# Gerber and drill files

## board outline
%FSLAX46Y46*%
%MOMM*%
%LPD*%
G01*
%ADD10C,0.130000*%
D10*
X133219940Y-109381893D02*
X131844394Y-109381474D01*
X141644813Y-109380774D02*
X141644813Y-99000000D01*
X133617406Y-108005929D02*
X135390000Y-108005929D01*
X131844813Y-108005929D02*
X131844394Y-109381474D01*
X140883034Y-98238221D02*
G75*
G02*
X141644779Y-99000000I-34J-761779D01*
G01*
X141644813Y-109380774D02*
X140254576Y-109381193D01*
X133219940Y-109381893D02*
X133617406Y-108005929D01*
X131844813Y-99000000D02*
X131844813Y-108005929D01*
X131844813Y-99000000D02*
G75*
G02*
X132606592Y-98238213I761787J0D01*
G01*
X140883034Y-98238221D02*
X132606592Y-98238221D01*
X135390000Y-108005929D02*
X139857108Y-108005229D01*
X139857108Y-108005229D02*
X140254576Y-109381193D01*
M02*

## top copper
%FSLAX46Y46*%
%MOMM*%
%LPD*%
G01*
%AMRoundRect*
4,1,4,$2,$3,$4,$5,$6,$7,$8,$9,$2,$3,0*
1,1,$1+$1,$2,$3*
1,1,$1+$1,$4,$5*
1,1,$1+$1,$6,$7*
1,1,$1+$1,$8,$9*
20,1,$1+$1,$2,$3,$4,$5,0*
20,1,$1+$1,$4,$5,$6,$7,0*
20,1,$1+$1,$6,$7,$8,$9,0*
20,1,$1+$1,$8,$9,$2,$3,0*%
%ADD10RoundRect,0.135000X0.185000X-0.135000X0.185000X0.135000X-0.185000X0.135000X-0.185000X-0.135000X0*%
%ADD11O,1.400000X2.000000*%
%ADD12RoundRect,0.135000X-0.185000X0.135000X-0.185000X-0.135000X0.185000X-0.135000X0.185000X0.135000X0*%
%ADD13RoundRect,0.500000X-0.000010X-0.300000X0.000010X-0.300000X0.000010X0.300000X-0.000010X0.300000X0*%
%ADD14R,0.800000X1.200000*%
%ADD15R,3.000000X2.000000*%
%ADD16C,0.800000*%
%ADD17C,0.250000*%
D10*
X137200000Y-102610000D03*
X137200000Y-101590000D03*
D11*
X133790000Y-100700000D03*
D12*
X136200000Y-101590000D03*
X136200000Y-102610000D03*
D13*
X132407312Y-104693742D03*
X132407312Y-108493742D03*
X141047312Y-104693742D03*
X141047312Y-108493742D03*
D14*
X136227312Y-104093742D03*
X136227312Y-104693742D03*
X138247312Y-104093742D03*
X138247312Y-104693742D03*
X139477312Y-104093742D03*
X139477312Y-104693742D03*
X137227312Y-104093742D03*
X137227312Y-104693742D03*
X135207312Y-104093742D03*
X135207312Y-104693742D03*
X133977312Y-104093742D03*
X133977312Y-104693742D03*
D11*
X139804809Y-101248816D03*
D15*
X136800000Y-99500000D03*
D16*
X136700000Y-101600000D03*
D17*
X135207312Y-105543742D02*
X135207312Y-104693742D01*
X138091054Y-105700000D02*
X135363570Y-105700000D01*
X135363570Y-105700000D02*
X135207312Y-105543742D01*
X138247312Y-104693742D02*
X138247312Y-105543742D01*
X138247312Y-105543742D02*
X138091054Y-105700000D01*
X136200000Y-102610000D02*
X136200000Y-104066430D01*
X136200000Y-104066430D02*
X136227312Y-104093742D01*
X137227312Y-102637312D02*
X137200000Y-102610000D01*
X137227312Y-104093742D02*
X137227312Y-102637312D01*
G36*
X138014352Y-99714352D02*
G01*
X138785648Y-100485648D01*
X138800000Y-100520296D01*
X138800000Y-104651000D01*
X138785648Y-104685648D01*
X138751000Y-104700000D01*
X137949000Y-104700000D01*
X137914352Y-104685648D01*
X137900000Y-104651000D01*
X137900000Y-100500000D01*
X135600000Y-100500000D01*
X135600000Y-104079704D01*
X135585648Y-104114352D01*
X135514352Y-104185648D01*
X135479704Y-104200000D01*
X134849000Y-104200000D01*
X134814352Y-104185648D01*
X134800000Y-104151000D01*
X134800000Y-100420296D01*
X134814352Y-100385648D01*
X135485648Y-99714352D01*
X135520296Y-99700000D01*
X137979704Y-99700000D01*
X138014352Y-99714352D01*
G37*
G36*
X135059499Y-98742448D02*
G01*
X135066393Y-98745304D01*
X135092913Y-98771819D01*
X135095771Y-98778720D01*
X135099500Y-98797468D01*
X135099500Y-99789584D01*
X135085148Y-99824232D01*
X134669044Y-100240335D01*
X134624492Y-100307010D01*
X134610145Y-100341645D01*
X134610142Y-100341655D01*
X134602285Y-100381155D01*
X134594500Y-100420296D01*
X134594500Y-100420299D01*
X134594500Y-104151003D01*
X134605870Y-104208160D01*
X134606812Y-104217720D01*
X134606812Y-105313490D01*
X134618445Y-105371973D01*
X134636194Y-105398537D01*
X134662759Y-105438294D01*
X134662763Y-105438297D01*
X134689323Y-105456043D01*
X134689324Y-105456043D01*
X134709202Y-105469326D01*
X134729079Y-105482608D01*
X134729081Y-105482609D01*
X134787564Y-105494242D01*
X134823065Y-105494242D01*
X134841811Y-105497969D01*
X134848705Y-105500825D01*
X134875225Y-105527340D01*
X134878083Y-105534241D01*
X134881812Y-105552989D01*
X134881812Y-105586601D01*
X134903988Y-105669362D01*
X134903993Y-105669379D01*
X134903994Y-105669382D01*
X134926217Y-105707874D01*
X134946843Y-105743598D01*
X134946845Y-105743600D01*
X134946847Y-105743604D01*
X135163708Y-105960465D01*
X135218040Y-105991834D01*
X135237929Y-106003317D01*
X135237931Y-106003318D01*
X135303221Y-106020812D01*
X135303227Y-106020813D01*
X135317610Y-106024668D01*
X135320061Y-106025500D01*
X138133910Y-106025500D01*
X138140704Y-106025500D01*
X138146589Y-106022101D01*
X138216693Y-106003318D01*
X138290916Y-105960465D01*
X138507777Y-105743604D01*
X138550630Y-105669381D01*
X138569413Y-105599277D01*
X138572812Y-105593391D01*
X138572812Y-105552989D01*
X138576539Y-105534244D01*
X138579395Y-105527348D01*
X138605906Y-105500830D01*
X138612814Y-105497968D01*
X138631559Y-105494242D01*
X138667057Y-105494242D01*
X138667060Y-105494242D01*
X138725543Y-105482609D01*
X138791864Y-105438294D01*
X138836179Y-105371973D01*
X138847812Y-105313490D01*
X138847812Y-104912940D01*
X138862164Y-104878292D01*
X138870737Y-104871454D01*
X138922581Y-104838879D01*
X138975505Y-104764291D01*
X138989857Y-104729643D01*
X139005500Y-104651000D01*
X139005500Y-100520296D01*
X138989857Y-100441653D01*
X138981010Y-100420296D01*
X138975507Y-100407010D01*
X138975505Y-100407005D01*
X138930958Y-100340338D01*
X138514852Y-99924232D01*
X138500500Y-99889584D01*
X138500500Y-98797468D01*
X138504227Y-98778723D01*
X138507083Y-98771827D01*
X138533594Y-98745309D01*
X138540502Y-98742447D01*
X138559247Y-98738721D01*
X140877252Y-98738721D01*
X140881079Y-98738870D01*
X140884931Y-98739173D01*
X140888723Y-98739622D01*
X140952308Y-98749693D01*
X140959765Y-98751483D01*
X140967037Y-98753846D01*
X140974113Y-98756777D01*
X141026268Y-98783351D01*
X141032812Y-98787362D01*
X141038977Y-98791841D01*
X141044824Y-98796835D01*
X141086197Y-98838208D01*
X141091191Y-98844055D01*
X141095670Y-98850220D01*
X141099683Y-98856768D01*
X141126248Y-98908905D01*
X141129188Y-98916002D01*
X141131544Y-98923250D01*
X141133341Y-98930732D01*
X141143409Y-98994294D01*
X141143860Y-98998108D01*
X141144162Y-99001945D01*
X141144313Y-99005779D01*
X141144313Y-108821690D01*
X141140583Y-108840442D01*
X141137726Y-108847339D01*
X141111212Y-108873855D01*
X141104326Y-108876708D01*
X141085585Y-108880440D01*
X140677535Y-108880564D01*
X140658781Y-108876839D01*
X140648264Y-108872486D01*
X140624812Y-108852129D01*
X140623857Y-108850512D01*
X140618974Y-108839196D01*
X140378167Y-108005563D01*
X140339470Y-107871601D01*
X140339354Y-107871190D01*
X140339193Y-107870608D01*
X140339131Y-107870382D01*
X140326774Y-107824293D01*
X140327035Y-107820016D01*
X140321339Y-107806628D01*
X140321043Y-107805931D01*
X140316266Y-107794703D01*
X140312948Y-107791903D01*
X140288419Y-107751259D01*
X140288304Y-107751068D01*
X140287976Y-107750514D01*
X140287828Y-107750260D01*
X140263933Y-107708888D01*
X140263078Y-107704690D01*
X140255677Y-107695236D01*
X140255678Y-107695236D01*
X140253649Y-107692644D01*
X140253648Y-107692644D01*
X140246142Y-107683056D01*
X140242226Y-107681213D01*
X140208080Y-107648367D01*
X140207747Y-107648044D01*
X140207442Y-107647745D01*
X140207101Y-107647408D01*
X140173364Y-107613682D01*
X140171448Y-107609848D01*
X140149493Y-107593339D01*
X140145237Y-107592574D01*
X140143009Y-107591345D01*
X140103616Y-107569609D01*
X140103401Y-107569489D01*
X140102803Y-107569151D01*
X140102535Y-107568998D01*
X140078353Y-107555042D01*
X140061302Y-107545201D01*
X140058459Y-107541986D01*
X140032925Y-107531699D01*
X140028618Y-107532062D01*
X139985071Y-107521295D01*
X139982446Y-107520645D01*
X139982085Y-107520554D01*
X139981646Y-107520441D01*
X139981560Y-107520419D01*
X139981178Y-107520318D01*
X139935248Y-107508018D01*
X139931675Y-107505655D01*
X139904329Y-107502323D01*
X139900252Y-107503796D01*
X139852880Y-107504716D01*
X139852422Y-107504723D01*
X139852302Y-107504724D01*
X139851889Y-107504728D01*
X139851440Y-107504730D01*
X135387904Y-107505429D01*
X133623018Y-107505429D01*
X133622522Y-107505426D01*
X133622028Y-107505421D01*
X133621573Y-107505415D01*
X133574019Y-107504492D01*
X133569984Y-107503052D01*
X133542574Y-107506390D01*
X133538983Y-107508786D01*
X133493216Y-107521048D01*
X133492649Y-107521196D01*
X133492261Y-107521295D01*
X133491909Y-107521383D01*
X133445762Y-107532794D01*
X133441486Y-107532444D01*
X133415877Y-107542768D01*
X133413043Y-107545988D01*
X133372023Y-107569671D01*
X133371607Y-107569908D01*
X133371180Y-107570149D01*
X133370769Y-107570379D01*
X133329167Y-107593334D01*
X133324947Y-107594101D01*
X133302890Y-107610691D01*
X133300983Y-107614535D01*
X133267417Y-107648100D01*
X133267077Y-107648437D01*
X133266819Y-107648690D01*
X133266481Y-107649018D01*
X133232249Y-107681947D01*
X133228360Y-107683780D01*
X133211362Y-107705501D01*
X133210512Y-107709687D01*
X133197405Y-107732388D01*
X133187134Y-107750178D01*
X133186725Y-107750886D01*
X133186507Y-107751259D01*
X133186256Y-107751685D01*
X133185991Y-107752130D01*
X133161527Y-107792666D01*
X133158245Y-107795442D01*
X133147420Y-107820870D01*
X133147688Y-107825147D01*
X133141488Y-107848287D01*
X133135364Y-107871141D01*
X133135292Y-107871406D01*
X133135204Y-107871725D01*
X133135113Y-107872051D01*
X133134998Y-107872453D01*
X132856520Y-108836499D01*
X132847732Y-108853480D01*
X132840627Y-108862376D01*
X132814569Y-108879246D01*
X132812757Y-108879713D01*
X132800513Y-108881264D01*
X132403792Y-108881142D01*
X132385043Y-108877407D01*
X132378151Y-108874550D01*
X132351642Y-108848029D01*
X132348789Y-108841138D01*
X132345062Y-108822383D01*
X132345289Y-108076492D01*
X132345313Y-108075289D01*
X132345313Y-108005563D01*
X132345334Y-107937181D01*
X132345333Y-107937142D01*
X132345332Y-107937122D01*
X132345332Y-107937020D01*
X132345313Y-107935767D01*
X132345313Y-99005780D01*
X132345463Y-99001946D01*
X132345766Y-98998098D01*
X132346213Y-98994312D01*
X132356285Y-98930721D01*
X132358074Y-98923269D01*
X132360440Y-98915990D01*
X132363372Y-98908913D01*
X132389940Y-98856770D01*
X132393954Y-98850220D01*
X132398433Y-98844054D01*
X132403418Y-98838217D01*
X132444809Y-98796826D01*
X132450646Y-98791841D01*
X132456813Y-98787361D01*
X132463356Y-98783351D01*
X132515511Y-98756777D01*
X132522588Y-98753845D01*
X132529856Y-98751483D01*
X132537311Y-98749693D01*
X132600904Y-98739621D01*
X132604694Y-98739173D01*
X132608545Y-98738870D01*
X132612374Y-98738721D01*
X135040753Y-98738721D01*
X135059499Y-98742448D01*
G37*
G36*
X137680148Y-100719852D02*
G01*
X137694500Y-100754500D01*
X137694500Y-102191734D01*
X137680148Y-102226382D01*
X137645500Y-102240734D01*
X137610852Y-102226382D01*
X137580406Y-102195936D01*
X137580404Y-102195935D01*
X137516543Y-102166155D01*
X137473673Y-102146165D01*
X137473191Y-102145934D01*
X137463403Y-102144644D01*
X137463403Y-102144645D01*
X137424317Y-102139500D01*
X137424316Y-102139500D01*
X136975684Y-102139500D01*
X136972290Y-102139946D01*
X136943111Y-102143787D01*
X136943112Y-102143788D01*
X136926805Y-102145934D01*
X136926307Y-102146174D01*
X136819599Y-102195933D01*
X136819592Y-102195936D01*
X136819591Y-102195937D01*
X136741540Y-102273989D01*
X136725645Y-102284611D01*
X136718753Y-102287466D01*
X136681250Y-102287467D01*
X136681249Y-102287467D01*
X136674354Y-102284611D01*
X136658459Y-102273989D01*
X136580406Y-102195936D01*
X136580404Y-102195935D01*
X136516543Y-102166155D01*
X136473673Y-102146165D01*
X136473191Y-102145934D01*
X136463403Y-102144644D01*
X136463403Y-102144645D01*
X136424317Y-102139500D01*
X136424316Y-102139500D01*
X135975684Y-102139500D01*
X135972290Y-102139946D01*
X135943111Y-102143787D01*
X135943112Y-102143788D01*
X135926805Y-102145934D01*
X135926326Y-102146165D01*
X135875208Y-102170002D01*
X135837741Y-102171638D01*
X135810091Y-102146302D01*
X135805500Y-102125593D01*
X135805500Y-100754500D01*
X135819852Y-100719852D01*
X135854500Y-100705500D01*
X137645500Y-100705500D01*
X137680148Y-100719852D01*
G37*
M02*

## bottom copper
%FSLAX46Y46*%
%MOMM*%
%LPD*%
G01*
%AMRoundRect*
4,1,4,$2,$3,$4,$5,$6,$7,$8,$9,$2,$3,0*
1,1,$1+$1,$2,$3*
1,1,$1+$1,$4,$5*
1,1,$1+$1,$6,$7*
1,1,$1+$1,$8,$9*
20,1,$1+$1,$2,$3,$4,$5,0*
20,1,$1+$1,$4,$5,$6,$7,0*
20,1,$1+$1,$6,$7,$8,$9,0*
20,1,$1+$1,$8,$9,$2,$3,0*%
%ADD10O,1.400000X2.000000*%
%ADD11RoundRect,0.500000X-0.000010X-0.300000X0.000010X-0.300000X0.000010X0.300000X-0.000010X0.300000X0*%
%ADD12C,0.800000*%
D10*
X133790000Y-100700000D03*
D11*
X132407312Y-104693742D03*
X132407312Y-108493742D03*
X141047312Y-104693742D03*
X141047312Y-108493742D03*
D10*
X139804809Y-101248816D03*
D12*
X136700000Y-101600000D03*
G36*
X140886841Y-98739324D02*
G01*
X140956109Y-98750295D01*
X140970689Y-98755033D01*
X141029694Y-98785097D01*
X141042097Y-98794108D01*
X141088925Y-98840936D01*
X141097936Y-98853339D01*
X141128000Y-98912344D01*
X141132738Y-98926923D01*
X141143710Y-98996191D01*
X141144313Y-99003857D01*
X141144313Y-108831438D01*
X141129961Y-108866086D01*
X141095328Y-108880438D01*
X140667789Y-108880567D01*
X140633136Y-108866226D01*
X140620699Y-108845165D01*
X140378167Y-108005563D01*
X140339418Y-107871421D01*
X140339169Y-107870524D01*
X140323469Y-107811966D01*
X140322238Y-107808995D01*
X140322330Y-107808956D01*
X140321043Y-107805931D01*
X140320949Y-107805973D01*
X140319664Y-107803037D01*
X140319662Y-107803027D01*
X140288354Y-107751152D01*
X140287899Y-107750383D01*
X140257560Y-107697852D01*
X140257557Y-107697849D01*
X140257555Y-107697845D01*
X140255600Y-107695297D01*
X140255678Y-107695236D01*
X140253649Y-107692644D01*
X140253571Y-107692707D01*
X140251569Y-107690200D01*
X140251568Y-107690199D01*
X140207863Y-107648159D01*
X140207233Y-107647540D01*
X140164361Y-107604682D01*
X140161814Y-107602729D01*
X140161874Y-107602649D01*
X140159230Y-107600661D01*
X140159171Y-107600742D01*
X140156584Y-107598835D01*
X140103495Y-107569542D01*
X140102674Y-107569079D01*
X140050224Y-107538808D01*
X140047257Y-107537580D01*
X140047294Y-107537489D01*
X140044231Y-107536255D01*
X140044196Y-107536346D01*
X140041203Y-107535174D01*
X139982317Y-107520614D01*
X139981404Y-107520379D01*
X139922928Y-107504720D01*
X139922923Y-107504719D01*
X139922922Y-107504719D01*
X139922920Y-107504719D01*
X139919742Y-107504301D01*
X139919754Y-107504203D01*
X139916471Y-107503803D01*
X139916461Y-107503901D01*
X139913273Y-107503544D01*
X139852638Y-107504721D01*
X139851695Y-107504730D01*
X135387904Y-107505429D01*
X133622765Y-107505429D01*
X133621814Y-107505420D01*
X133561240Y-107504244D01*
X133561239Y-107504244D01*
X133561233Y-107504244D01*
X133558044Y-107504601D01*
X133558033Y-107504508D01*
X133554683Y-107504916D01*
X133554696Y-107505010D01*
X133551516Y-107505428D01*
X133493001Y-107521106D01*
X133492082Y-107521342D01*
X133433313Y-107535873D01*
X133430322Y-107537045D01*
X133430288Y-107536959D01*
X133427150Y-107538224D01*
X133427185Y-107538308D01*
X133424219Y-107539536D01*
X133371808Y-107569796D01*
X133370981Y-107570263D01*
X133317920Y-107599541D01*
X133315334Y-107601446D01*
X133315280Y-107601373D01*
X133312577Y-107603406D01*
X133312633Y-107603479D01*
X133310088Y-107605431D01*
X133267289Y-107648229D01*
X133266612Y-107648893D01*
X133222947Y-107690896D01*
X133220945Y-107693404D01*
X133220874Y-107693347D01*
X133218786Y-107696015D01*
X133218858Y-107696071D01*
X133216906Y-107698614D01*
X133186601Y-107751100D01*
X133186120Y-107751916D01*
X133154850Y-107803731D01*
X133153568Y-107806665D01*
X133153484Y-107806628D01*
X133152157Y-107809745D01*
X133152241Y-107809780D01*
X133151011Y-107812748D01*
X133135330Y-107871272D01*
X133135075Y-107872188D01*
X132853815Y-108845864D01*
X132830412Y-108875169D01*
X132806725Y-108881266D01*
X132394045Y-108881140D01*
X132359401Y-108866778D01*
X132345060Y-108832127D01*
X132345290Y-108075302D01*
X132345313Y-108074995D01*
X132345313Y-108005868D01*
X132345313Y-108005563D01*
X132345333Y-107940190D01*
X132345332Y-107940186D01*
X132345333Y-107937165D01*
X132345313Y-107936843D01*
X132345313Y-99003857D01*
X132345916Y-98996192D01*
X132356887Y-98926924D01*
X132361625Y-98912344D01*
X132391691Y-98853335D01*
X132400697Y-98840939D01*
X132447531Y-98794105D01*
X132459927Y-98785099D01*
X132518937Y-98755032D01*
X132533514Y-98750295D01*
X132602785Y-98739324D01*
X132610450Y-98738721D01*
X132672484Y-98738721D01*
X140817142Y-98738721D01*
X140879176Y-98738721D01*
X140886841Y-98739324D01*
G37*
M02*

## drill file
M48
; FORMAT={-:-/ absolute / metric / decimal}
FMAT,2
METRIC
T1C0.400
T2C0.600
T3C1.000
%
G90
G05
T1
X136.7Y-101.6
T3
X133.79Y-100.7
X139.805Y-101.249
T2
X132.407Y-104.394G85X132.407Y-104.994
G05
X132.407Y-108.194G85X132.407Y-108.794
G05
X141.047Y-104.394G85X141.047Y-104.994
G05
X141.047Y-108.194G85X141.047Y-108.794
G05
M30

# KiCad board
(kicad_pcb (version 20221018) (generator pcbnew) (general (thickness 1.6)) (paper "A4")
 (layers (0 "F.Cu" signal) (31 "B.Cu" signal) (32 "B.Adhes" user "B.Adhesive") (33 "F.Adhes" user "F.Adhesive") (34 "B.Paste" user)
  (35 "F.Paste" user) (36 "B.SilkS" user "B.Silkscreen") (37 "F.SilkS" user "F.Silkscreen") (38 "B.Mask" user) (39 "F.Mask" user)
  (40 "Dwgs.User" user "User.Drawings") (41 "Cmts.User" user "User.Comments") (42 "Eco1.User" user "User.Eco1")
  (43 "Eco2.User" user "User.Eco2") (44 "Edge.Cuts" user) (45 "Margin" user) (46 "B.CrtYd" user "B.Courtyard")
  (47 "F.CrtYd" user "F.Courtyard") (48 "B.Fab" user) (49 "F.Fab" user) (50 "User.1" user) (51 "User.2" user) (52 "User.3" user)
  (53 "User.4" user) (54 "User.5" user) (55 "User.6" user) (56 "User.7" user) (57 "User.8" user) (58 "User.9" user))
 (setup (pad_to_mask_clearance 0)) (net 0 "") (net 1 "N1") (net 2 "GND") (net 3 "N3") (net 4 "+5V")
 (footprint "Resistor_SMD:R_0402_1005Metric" (layer "F.Cu") (at 137.2 102.1 90)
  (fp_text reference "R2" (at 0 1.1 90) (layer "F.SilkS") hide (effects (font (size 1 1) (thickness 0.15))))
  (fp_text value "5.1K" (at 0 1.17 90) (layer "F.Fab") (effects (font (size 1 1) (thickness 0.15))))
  (pad "1" smd roundrect (at -0.51 0 90) (size 0.54 0.64) (layers "F.Cu" "F.Paste" "F.Mask") (roundrect_rratio 0.25) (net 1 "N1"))
  (pad "2" smd roundrect (at 0.51 0 90) (size 0.54 0.64) (layers "F.Cu" "F.Paste" "F.Mask") (roundrect_rratio 0.25) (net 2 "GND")))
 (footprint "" (layer "F.Cu") (at 133.79 100.7 -90)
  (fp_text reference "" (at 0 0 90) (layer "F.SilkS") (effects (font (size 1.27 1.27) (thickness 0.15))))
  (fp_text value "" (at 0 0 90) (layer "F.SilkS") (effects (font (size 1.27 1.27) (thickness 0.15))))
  (pad "1" thru_hole oval (at 0 0 90) (size 2 1.4) (drill 1) (layers "*.Cu" "*.Mask") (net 2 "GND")))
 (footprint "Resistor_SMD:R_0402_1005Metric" (layer "F.Cu") (at 136.2 102.1 -90)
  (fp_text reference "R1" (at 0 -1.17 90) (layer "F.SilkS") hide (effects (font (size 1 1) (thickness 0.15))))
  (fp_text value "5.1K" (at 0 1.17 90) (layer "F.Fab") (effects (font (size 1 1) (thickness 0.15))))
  (pad "1" smd roundrect (at -0.51 0 270) (size 0.54 0.64) (layers "F.Cu" "F.Paste" "F.Mask") (roundrect_rratio 0.25) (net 2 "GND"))
  (pad "2" smd roundrect (at 0.51 0 270) (size 0.54 0.64) (layers "F.Cu" "F.Paste" "F.Mask") (roundrect_rratio 0.25) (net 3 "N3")))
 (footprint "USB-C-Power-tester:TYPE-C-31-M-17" (layer "F.Cu") (at 136.727312 108.493742)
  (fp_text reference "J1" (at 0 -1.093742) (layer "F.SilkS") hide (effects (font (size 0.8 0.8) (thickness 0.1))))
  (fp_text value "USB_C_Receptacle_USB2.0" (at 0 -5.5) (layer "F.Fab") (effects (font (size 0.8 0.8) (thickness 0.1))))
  (pad "1" thru_hole roundrect (at -4.32 -3.8) (size 1 1.6) (drill oval 0.6 1.2) (layers "*.Cu" "*.Mask") (roundrect_rratio 0.5)
   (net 2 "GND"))
  (pad "1" thru_hole roundrect (at -4.32 0) (size 1 1.6) (drill oval 0.6 1.2) (layers "*.Cu" "*.Mask") (roundrect_rratio 0.5) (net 2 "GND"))
  (pad "1" thru_hole roundrect (at 4.32 -3.8) (size 1 1.6) (drill oval 0.6 1.2) (layers "*.Cu" "*.Mask") (roundrect_rratio 0.5)
   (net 2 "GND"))
  (pad "1" thru_hole roundrect (at 4.32 0) (size 1 1.6) (drill oval 0.6 1.2) (layers "*.Cu" "*.Mask") (roundrect_rratio 0.5) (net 2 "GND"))
  (pad "A5" smd rect (at -0.5 -4.4) (size 0.8 1.2) (layers "F.Cu" "F.Paste" "F.Mask") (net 3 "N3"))
  (pad "A5" smd rect (at -0.5 -3.8) (size 0.8 1.2) (layers "F.Cu" "F.Paste" "F.Mask") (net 3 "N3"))
  (pad "A9" smd rect (at 1.52 -4.4) (size 0.8 1.2) (layers "F.Cu" "F.Paste" "F.Mask") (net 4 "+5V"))
  (pad "A9" smd rect (at 1.52 -3.8) (size 0.8 1.2) (layers "F.Cu" "F.Paste" "F.Mask") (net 4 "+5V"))
  (pad "A12" smd rect (at 2.75 -4.4) (size 0.8 1.2) (layers "F.Cu" "F.Paste" "F.Mask") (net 2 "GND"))
  (pad "A12" smd rect (at 2.75 -3.8) (size 0.8 1.2) (layers "F.Cu" "F.Paste" "F.Mask") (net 2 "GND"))
  (pad "B5" smd rect (at 0.5 -4.4) (size 0.8 1.2) (layers "F.Cu" "F.Paste" "F.Mask") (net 1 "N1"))
  (pad "B5" smd rect (at 0.5 -3.8) (size 0.8 1.2) (layers "F.Cu" "F.Paste" "F.Mask") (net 1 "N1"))
  (pad "B9" smd rect (at -1.52 -4.4) (size 0.8 1.2) (layers "F.Cu" "F.Paste" "F.Mask") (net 4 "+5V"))
  (pad "B9" smd rect (at -1.52 -3.8) (size 0.8 1.2) (layers "F.Cu" "F.Paste" "F.Mask") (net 4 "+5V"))
  (pad "B12" smd rect (at -2.75 -4.4) (size 0.8 1.2) (layers "F.Cu" "F.Paste" "F.Mask") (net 2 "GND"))
  (pad "B12" smd rect (at -2.75 -3.8) (size 0.8 1.2) (layers "F.Cu" "F.Paste" "F.Mask") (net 2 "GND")))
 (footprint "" (layer "F.Cu") (at 139.804809 101.248816 -90)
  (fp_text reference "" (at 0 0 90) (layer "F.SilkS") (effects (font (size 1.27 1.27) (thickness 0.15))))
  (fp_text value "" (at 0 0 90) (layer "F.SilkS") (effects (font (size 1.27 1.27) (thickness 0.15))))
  (pad "1" thru_hole oval (at 0 0 270) (size 2 1.4) (drill 1) (layers "*.Cu" "*.Mask") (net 2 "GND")))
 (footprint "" (layer "F.Cu") (at 136.8 99.5 90)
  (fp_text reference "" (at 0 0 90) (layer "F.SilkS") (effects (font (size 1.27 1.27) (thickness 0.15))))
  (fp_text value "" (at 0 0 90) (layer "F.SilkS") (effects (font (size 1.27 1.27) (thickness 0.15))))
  (pad "" smd rect (at 0 0 90) (size 2 3) (layers "F.Cu" "F.Paste" "F.Mask") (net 4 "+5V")))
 (gr_line (start 133.21994 109.381893) (end 131.844394 109.381474) (stroke (width 0.13) (type solid)) (layer "Edge.Cuts"))
 (gr_line (start 141.644813 109.380774) (end 141.644813 99) (stroke (width 0.13) (type solid)) (layer "Edge.Cuts"))
 (gr_line (start 133.617406 108.005929) (end 135.39 108.005929) (stroke (width 0.13) (type solid)) (layer "Edge.Cuts"))
 (gr_line (start 131.844813 108.005929) (end 131.844394 109.381474) (stroke (width 0.13) (type solid)) (layer "Edge.Cuts"))
 (gr_arc (start 140.883034 98.238221) (mid 141.421693 98.461341) (end 141.644813 99) (stroke (width 0.13) (type default))
  (layer "Edge.Cuts"))
 (gr_line (start 141.644813 109.380774) (end 140.254576 109.381193) (stroke (width 0.13) (type solid)) (layer "Edge.Cuts"))
 (gr_line (start 133.21994 109.381893) (end 133.617406 108.005929) (stroke (width 0.13) (type solid)) (layer "Edge.Cuts"))
 (gr_line (start 131.844813 99) (end 131.844813 108.005929) (stroke (width 0.13) (type solid)) (layer "Edge.Cuts"))
 (gr_arc (start 131.844813 99) (mid 132.067933 98.461341) (end 132.606592 98.238221) (stroke (width 0.13) (type default))
  (layer "Edge.Cuts"))
 (gr_line (start 140.883034 98.238221) (end 132.606592 98.238221) (stroke (width 0.13) (type solid)) (layer "Edge.Cuts"))
 (gr_line (start 135.39 108.005929) (end 139.857108 108.005229) (stroke (width 0.13) (type solid)) (layer "Edge.Cuts"))
 (gr_line (start 139.857108 108.005229) (end 140.254576 109.381193) (stroke (width 0.13) (type solid)) (layer "Edge.Cuts"))
 (via (at 136.7 101.6) (size 0.8) (drill 0.4) (layers "F.Cu" "B.Cu") (free) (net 2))
 (segment (start 135.207312 105.543742) (end 135.207312 104.693742) (width 0.25) (layer "F.Cu") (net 4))
 (segment (start 138.091054 105.7) (end 135.36357 105.7) (width 0.25) (layer "F.Cu") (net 4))
 (segment (start 135.36357 105.7) (end 135.207312 105.543742) (width 0.25) (layer "F.Cu") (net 4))
 (segment (start 138.247312 104.693742) (end 138.247312 105.543742) (width 0.25) (layer "F.Cu") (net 4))
 (segment (start 138.247312 105.543742) (end 138.091054 105.7) (width 0.25) (layer "F.Cu") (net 4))
 (segment (start 136.2 102.61) (end 136.2 104.06643) (width 0.25) (layer "F.Cu") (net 3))
 (segment (start 136.2 104.06643) (end 136.227312 104.093742) (width 0.25) (layer "F.Cu") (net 3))
 (segment (start 137.227312 102.637312) (end 137.2 102.61) (width 0.25) (layer "F.Cu") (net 1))
 (segment (start 137.227312 104.093742) (end 137.227312 102.637312) (width 0.25) (layer "F.Cu") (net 1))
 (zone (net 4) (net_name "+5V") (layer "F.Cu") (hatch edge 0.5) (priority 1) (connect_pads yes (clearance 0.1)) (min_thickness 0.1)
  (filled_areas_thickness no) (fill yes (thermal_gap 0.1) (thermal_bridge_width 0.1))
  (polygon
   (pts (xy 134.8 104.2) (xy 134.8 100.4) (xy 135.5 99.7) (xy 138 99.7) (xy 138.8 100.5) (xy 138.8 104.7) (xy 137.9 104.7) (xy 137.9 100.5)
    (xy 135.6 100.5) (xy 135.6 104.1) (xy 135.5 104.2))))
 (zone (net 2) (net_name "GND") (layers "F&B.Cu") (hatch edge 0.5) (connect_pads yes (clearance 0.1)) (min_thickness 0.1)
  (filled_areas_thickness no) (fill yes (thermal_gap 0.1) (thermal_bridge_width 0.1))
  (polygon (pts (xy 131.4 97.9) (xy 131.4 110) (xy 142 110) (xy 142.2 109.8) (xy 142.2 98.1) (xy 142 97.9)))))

